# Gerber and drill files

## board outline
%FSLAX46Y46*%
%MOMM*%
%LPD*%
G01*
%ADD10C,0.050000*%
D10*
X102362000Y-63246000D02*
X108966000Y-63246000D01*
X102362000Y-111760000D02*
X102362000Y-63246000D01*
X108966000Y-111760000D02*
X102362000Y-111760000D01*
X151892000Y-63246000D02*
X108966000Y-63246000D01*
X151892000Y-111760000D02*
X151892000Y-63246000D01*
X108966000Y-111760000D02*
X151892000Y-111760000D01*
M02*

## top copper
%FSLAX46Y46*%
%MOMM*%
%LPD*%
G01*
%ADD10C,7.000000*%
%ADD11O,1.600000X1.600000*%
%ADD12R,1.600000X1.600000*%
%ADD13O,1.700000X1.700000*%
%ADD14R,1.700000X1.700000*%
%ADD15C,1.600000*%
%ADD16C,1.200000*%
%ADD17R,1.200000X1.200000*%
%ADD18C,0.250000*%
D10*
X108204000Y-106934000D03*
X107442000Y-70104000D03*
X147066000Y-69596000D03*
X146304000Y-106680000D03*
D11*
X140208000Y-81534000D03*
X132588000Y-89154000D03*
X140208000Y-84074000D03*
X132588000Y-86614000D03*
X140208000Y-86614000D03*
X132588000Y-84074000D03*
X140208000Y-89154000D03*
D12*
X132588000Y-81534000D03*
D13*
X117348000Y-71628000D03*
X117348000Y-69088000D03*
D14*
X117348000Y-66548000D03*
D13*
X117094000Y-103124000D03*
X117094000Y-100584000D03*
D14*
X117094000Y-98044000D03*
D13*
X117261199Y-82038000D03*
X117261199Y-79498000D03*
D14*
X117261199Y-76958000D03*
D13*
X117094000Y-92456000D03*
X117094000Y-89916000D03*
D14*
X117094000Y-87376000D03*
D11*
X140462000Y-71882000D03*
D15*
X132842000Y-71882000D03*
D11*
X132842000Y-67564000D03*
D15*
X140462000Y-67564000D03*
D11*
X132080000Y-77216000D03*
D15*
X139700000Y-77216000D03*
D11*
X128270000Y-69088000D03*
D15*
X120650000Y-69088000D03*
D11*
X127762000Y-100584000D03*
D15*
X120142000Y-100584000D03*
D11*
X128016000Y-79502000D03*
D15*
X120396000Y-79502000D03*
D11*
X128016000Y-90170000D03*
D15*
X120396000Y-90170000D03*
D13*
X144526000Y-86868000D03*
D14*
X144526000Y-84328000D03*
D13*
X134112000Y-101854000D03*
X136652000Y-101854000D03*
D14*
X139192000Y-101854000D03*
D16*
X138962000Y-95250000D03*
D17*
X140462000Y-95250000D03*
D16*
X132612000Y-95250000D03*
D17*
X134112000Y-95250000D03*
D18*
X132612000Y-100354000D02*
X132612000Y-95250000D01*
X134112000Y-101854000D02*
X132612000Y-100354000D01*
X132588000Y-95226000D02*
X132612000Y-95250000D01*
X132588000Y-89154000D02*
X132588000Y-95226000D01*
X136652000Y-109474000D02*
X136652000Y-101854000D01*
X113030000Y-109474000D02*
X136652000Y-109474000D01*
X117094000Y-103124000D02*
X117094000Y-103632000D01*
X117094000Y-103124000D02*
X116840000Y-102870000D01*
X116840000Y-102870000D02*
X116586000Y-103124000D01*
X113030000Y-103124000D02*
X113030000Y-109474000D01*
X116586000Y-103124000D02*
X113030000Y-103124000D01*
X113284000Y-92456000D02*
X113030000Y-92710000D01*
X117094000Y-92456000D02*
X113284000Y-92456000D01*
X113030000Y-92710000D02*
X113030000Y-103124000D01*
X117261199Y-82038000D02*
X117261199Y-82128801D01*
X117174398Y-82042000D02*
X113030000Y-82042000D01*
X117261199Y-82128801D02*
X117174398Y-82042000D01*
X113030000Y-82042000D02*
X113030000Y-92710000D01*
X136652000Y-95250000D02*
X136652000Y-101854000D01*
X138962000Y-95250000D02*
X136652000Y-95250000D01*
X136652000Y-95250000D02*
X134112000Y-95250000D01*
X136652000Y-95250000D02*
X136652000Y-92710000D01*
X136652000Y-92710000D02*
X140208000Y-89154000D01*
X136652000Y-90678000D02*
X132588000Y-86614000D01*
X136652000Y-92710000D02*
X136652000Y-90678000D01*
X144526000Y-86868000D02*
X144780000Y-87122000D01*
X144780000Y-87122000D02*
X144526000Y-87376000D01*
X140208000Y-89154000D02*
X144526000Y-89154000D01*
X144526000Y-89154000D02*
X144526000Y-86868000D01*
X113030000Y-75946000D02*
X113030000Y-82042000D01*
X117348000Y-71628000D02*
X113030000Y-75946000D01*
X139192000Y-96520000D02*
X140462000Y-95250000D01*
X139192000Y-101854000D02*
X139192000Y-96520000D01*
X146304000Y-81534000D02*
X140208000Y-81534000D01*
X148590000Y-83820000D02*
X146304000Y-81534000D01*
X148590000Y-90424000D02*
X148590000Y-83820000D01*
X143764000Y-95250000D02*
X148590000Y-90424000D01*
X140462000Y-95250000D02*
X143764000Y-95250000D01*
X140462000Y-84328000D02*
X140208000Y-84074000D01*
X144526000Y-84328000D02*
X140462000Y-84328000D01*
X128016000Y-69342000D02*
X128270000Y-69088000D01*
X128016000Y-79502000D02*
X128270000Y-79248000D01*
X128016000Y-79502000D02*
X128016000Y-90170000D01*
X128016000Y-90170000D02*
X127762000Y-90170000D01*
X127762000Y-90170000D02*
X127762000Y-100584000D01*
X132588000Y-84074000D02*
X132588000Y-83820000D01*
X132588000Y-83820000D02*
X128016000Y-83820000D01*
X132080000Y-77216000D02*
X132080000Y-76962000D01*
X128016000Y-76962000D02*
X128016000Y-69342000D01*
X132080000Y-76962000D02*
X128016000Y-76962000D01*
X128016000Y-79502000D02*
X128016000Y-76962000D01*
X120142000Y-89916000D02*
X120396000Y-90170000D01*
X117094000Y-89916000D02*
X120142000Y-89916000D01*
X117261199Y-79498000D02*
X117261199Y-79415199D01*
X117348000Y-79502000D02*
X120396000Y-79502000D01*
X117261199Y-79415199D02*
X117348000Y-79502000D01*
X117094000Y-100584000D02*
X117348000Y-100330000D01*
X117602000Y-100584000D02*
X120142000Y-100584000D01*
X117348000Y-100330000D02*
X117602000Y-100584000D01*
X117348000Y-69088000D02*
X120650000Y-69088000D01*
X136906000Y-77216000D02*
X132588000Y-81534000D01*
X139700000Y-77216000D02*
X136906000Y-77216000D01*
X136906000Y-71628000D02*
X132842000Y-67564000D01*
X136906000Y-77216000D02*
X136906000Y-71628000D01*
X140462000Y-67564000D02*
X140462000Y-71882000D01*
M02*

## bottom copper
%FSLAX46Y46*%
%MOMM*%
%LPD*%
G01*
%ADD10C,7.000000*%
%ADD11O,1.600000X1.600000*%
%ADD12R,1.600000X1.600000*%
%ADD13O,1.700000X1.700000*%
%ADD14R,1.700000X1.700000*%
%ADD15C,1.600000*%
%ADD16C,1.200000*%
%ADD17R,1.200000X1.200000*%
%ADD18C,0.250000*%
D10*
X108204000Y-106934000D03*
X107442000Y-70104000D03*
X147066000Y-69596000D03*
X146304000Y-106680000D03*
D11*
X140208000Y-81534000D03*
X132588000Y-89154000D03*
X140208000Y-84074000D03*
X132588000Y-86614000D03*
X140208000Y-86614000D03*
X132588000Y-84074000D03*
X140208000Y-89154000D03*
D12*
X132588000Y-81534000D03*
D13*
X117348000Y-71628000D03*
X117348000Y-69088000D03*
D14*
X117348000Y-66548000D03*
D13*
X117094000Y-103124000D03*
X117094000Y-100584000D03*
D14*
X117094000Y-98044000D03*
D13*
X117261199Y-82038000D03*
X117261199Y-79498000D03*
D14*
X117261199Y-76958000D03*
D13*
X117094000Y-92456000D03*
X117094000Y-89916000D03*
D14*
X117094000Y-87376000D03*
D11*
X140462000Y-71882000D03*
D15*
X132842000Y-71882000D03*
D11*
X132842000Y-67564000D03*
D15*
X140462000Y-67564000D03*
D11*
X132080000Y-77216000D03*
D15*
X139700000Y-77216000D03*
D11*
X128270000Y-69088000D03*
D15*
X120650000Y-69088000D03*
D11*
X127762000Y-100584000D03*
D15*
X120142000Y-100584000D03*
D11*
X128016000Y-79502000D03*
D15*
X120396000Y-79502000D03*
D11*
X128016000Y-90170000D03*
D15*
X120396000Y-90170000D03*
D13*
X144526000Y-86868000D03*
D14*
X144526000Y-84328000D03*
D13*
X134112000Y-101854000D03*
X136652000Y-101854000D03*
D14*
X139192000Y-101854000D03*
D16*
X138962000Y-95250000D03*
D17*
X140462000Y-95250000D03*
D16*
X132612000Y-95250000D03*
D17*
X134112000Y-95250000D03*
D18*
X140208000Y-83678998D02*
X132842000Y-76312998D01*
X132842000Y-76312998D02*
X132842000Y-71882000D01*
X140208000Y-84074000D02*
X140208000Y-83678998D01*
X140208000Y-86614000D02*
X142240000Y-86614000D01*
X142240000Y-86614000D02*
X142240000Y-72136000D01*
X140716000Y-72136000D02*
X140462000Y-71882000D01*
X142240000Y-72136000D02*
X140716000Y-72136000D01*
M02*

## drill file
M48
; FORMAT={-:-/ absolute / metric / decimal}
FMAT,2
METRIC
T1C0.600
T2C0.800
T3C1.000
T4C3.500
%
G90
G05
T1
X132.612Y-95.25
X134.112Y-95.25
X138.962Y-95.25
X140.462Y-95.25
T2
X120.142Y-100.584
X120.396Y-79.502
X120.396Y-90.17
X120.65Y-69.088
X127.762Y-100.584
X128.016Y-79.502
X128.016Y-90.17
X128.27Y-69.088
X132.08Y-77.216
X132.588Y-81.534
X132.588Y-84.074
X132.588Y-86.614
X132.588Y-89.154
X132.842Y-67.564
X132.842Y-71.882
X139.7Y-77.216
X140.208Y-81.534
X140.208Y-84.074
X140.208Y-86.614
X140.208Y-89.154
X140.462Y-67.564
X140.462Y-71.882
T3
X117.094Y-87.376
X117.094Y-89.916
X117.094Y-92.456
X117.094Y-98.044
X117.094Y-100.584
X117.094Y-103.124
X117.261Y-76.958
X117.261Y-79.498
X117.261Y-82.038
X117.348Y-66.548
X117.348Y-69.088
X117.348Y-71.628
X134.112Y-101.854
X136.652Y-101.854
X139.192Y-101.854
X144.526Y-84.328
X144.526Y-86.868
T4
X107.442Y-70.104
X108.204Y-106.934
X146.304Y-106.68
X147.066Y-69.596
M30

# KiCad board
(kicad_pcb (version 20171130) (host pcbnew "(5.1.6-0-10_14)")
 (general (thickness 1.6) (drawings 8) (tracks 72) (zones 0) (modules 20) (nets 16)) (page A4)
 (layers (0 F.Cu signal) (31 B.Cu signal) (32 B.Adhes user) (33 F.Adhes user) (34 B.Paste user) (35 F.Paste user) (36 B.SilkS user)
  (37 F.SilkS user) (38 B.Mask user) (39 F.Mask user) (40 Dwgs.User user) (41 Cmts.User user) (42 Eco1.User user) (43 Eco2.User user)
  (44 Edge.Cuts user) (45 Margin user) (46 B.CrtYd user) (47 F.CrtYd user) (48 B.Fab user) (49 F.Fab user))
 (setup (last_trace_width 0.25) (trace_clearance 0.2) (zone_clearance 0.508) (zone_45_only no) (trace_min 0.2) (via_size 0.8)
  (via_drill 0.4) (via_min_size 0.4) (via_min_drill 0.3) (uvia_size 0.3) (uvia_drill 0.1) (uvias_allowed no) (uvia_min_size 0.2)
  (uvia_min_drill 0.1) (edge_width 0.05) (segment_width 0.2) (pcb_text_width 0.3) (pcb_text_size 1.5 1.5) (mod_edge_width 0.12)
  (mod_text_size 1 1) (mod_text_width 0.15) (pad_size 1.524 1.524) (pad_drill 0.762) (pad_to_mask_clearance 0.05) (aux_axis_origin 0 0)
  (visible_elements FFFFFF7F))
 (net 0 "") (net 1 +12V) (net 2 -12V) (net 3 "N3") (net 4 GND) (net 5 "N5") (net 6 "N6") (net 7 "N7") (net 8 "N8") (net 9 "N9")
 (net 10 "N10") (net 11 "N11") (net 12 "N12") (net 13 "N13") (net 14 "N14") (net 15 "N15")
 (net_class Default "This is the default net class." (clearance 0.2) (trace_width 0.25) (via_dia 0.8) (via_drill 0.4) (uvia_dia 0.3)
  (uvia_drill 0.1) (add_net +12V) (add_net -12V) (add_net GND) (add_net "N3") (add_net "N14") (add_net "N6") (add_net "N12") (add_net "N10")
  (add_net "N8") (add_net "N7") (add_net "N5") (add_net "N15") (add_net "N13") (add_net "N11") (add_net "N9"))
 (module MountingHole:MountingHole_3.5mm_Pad (layer F.Cu) (at 108.204 106.934)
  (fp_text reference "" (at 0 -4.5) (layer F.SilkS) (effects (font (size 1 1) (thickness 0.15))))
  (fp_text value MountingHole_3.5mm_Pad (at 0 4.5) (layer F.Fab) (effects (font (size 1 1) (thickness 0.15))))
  (pad 1 thru_hole circle (at 0 0) (size 7 7) (drill 3.5) (layers *.Cu *.Mask)))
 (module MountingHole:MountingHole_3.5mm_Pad (layer F.Cu) (at 107.442 70.104)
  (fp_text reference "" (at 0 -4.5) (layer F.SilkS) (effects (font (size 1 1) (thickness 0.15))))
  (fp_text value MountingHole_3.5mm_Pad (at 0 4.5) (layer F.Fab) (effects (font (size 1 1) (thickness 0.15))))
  (pad 1 thru_hole circle (at 0 0) (size 7 7) (drill 3.5) (layers *.Cu *.Mask)))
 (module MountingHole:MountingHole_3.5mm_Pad (layer F.Cu) (at 147.066 69.596)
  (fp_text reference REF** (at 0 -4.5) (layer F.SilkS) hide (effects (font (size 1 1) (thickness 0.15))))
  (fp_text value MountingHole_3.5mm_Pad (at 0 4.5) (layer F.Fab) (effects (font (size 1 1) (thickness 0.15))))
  (pad 1 thru_hole circle (at 0 0) (size 7 7) (drill 3.5) (layers *.Cu *.Mask)))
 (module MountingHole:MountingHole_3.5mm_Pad (layer F.Cu) (at 146.304 106.68)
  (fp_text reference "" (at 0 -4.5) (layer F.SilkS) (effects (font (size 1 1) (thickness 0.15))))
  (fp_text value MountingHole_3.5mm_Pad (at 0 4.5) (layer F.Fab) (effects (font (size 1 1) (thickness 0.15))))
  (pad 1 thru_hole circle (at 0 0) (size 7 7) (drill 3.5) (layers *.Cu *.Mask)))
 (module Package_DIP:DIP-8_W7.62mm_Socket (layer F.Cu) (at 132.588 81.534)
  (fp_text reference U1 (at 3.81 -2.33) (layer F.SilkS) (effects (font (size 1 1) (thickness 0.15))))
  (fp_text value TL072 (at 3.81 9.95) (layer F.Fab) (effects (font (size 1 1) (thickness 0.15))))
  (pad 8 thru_hole oval (at 7.62 0) (size 1.6 1.6) (drill 0.8) (layers *.Cu *.Mask) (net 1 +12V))
  (pad 4 thru_hole oval (at 0 7.62) (size 1.6 1.6) (drill 0.8) (layers *.Cu *.Mask) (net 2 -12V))
  (pad 7 thru_hole oval (at 7.62 2.54) (size 1.6 1.6) (drill 0.8) (layers *.Cu *.Mask) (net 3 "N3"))
  (pad 3 thru_hole oval (at 0 5.08) (size 1.6 1.6) (drill 0.8) (layers *.Cu *.Mask) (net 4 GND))
  (pad 6 thru_hole oval (at 7.62 5.08) (size 1.6 1.6) (drill 0.8) (layers *.Cu *.Mask) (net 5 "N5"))
  (pad 2 thru_hole oval (at 0 2.54) (size 1.6 1.6) (drill 0.8) (layers *.Cu *.Mask) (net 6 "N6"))
  (pad 5 thru_hole oval (at 7.62 7.62) (size 1.6 1.6) (drill 0.8) (layers *.Cu *.Mask) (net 4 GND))
  (pad 1 thru_hole rect (at 0 0) (size 1.6 1.6) (drill 0.8) (layers *.Cu *.Mask) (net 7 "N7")))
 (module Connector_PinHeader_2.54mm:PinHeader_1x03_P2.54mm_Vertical (layer F.Cu) (at 117.348 66.548)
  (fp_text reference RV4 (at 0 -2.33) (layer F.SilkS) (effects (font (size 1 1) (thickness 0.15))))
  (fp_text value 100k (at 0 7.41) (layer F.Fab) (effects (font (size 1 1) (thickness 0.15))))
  (pad 3 thru_hole oval (at 0 5.08) (size 1.7 1.7) (drill 1) (layers *.Cu *.Mask) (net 4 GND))
  (pad 2 thru_hole oval (at 0 2.54) (size 1.7 1.7) (drill 1) (layers *.Cu *.Mask) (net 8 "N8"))
  (pad 1 thru_hole rect (at 0 0) (size 1.7 1.7) (drill 1) (layers *.Cu *.Mask) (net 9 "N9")))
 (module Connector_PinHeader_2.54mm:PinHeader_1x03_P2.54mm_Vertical (layer F.Cu) (at 117.094 98.044)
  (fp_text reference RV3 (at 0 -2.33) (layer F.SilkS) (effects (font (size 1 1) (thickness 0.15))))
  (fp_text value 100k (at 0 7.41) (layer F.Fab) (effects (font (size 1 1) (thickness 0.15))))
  (pad 3 thru_hole oval (at 0 5.08) (size 1.7 1.7) (drill 1) (layers *.Cu *.Mask) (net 4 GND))
  (pad 2 thru_hole oval (at 0 2.54) (size 1.7 1.7) (drill 1) (layers *.Cu *.Mask) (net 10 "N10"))
  (pad 1 thru_hole rect (at 0 0) (size 1.7 1.7) (drill 1) (layers *.Cu *.Mask) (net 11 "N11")))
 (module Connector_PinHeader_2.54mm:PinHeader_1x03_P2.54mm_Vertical (layer F.Cu) (at 117.261199 76.958)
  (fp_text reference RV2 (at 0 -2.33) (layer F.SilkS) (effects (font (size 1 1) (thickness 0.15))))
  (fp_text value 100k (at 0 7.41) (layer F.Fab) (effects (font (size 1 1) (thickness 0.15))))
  (pad 3 thru_hole oval (at 0 5.08) (size 1.7 1.7) (drill 1) (layers *.Cu *.Mask) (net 4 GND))
  (pad 2 thru_hole oval (at 0 2.54) (size 1.7 1.7) (drill 1) (layers *.Cu *.Mask) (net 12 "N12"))
  (pad 1 thru_hole rect (at 0 0) (size 1.7 1.7) (drill 1) (layers *.Cu *.Mask) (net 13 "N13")))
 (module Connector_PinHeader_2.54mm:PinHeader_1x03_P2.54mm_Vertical (layer F.Cu) (at 117.094 87.376)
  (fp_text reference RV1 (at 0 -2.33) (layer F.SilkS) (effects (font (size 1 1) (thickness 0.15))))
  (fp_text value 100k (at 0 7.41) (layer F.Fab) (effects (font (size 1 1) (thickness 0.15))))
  (pad 3 thru_hole oval (at 0 5.08) (size 1.7 1.7) (drill 1) (layers *.Cu *.Mask) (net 4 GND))
  (pad 2 thru_hole oval (at 0 2.54) (size 1.7 1.7) (drill 1) (layers *.Cu *.Mask) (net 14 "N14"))
  (pad 1 thru_hole rect (at 0 0) (size 1.7 1.7) (drill 1) (layers *.Cu *.Mask) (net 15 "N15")))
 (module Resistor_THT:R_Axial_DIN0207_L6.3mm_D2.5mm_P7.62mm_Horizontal (layer F.Cu) (at 132.842 71.882)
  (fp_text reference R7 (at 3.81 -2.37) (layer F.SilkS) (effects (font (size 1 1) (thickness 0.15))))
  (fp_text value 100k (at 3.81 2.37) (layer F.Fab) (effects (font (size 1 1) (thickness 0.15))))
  (pad 2 thru_hole oval (at 7.62 0) (size 1.6 1.6) (drill 0.8) (layers *.Cu *.Mask) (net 5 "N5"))
  (pad 1 thru_hole circle (at 0 0) (size 1.6 1.6) (drill 0.8) (layers *.Cu *.Mask) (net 3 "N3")))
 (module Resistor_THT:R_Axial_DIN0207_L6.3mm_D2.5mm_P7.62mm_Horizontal (layer F.Cu) (at 140.462 67.564 180)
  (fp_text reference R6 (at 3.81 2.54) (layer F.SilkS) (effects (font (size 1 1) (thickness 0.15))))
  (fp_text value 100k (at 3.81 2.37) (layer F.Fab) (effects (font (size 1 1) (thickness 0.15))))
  (pad 2 thru_hole oval (at 7.62 0 180) (size 1.6 1.6) (drill 0.8) (layers *.Cu *.Mask) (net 7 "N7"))
  (pad 1 thru_hole circle (at 0 0 180) (size 1.6 1.6) (drill 0.8) (layers *.Cu *.Mask) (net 5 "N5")))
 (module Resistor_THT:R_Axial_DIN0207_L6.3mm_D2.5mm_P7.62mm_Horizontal (layer F.Cu) (at 139.7 77.216 180)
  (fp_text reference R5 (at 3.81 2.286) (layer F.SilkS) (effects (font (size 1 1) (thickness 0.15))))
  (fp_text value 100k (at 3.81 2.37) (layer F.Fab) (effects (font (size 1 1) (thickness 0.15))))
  (pad 2 thru_hole oval (at 7.62 0 180) (size 1.6 1.6) (drill 0.8) (layers *.Cu *.Mask) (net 6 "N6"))
  (pad 1 thru_hole circle (at 0 0 180) (size 1.6 1.6) (drill 0.8) (layers *.Cu *.Mask) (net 7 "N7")))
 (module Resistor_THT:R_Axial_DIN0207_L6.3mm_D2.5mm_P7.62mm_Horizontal (layer F.Cu) (at 120.65 69.088)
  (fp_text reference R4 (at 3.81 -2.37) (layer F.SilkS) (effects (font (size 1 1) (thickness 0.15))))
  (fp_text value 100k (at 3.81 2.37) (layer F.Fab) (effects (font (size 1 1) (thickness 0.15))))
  (pad 2 thru_hole oval (at 7.62 0) (size 1.6 1.6) (drill 0.8) (layers *.Cu *.Mask) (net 6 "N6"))
  (pad 1 thru_hole circle (at 0 0) (size 1.6 1.6) (drill 0.8) (layers *.Cu *.Mask) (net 8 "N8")))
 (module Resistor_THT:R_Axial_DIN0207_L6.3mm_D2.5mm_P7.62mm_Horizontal (layer F.Cu) (at 120.142 100.584)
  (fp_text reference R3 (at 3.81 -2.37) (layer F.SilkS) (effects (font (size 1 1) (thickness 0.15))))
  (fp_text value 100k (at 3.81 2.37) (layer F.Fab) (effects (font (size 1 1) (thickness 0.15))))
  (pad 2 thru_hole oval (at 7.62 0) (size 1.6 1.6) (drill 0.8) (layers *.Cu *.Mask) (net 6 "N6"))
  (pad 1 thru_hole circle (at 0 0) (size 1.6 1.6) (drill 0.8) (layers *.Cu *.Mask) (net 10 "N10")))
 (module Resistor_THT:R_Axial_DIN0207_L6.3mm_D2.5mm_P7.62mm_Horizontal (layer F.Cu) (at 120.396 79.502)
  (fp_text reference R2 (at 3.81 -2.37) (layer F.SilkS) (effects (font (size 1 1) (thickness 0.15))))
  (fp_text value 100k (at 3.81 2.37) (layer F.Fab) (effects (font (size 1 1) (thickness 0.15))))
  (pad 2 thru_hole oval (at 7.62 0) (size 1.6 1.6) (drill 0.8) (layers *.Cu *.Mask) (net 6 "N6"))
  (pad 1 thru_hole circle (at 0 0) (size 1.6 1.6) (drill 0.8) (layers *.Cu *.Mask) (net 12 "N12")))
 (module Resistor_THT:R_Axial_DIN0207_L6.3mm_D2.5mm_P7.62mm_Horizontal (layer F.Cu) (at 120.396 90.17)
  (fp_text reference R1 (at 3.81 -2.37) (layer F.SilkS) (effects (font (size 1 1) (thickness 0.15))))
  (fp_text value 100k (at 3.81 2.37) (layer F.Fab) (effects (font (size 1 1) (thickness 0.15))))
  (pad 2 thru_hole oval (at 7.62 0) (size 1.6 1.6) (drill 0.8) (layers *.Cu *.Mask) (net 6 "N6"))
  (pad 1 thru_hole circle (at 0 0) (size 1.6 1.6) (drill 0.8) (layers *.Cu *.Mask) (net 14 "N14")))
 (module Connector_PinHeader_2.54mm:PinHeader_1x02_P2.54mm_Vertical (layer F.Cu) (at 144.526 84.328)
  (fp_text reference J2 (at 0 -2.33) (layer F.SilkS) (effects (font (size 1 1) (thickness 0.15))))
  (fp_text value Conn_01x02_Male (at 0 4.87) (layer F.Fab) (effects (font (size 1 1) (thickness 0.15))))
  (pad 2 thru_hole oval (at 0 2.54) (size 1.7 1.7) (drill 1) (layers *.Cu *.Mask) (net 4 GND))
  (pad 1 thru_hole rect (at 0 0) (size 1.7 1.7) (drill 1) (layers *.Cu *.Mask) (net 3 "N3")))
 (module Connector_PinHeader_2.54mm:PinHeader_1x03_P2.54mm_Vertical (layer F.Cu) (at 139.192 101.854 270)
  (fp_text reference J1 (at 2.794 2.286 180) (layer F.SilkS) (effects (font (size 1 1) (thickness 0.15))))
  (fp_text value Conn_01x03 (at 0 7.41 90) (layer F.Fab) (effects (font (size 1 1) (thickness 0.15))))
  (pad 3 thru_hole oval (at 0 5.08 270) (size 1.7 1.7) (drill 1) (layers *.Cu *.Mask) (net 2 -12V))
  (pad 2 thru_hole oval (at 0 2.54 270) (size 1.7 1.7) (drill 1) (layers *.Cu *.Mask) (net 4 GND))
  (pad 1 thru_hole rect (at 0 0 270) (size 1.7 1.7) (drill 1) (layers *.Cu *.Mask) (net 1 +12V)))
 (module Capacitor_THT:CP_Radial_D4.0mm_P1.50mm (layer F.Cu) (at 140.462 95.25 180)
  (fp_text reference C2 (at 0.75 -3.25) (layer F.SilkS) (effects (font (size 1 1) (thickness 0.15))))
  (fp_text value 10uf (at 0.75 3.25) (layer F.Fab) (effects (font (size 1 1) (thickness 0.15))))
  (pad 2 thru_hole circle (at 1.5 0 180) (size 1.2 1.2) (drill 0.6) (layers *.Cu *.Mask) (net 4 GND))
  (pad 1 thru_hole rect (at 0 0 180) (size 1.2 1.2) (drill 0.6) (layers *.Cu *.Mask) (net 1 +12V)))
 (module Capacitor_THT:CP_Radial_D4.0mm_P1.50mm (layer F.Cu) (at 134.112 95.25 180)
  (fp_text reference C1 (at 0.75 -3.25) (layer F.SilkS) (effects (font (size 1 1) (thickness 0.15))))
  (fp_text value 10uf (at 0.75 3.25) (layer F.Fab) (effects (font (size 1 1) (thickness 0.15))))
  (pad 2 thru_hole circle (at 1.5 0 180) (size 1.2 1.2) (drill 0.6) (layers *.Cu *.Mask) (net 2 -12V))
  (pad 1 thru_hole rect (at 0 0 180) (size 1.2 1.2) (drill 0.6) (layers *.Cu *.Mask) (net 4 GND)))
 (gr_line (start 102.362 63.246) (end 108.966 63.246) (layer Edge.Cuts) (width 0.05))
 (gr_line (start 102.362 111.76) (end 102.362 63.246) (layer Edge.Cuts) (width 0.05))
 (gr_line (start 108.966 111.76) (end 102.362 111.76) (layer Edge.Cuts) (width 0.05))
 (gr_line (start 151.892 63.246) (end 108.966 63.246) (layer Edge.Cuts) (width 0.05))
 (gr_line (start 151.892 111.76) (end 151.892 63.246) (layer Edge.Cuts) (width 0.05))
 (gr_line (start 108.966 111.76) (end 151.892 111.76) (layer Edge.Cuts) (width 0.05))
 (segment (start 132.612 100.354) (end 132.612 95.25) (width 0.25) (layer F.Cu) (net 2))
 (segment (start 134.112 101.854) (end 132.612 100.354) (width 0.25) (layer F.Cu) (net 2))
 (segment (start 132.588 95.226) (end 132.612 95.25) (width 0.25) (layer F.Cu) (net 2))
 (segment (start 132.588 89.154) (end 132.588 95.226) (width 0.25) (layer F.Cu) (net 2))
 (segment (start 136.652 109.474) (end 136.652 101.854) (width 0.25) (layer F.Cu) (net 4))
 (segment (start 113.03 109.474) (end 136.652 109.474) (width 0.25) (layer F.Cu) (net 4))
 (segment (start 117.094 103.124) (end 117.094 103.632) (width 0.25) (layer F.Cu) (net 4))
 (segment (start 117.094 103.124) (end 116.84 102.87) (width 0.25) (layer F.Cu) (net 4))
 (segment (start 116.84 102.87) (end 116.586 103.124) (width 0.25) (layer F.Cu) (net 4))
 (segment (start 113.03 103.124) (end 113.03 109.474) (width 0.25) (layer F.Cu) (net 4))
 (segment (start 116.586 103.124) (end 113.03 103.124) (width 0.25) (layer F.Cu) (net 4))
 (segment (start 113.284 92.456) (end 113.03 92.71) (width 0.25) (layer F.Cu) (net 4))
 (segment (start 117.094 92.456) (end 113.284 92.456) (width 0.25) (layer F.Cu) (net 4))
 (segment (start 113.03 92.71) (end 113.03 103.124) (width 0.25) (layer F.Cu) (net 4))
 (segment (start 117.261199 82.038) (end 117.261199 82.128801) (width 0.25) (layer F.Cu) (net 4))
 (segment (start 117.174398 82.042) (end 113.03 82.042) (width 0.25) (layer F.Cu) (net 4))
 (segment (start 117.261199 82.128801) (end 117.174398 82.042) (width 0.25) (layer F.Cu) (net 4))
 (segment (start 113.03 82.042) (end 113.03 92.71) (width 0.25) (layer F.Cu) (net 4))
 (segment (start 136.652 95.25) (end 136.652 101.854) (width 0.25) (layer F.Cu) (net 4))
 (segment (start 138.962 95.25) (end 136.652 95.25) (width 0.25) (layer F.Cu) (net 4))
 (segment (start 136.652 95.25) (end 134.112 95.25) (width 0.25) (layer F.Cu) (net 4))
 (segment (start 136.652 95.25) (end 136.652 92.71) (width 0.25) (layer F.Cu) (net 4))
 (segment (start 136.652 92.71) (end 140.208 89.154) (width 0.25) (layer F.Cu) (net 4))
 (segment (start 136.652 90.678) (end 132.588 86.614) (width 0.25) (layer F.Cu) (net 4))
 (segment (start 136.652 92.71) (end 136.652 90.678) (width 0.25) (layer F.Cu) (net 4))
 (segment (start 144.526 86.868) (end 144.78 87.122) (width 0.25) (layer F.Cu) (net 4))
 (segment (start 144.78 87.122) (end 144.526 87.376) (width 0.25) (layer F.Cu) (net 4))
 (segment (start 140.208 89.154) (end 144.526 89.154) (width 0.25) (layer F.Cu) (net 4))
 (segment (start 144.526 89.154) (end 144.526 86.868) (width 0.25) (layer F.Cu) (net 4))
 (segment (start 113.03 75.946) (end 113.03 82.042) (width 0.25) (layer F.Cu) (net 4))
 (segment (start 117.348 71.628) (end 113.03 75.946) (width 0.25) (layer F.Cu) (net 4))
 (segment (start 139.192 96.52) (end 140.462 95.25) (width 0.25) (layer F.Cu) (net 1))
 (segment (start 139.192 101.854) (end 139.192 96.52) (width 0.25) (layer F.Cu) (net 1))
 (segment (start 146.304 81.534) (end 140.208 81.534) (width 0.25) (layer F.Cu) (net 1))
 (segment (start 148.59 83.82) (end 146.304 81.534) (width 0.25) (layer F.Cu) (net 1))
 (segment (start 148.59 90.424) (end 148.59 83.82) (width 0.25) (layer F.Cu) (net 1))
 (segment (start 143.764 95.25) (end 148.59 90.424) (width 0.25) (layer F.Cu) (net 1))
 (segment (start 140.462 95.25) (end 143.764 95.25) (width 0.25) (layer F.Cu) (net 1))
 (segment (start 140.462 84.328) (end 140.208 84.074) (width 0.25) (layer F.Cu) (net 3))
 (segment (start 144.526 84.328) (end 140.462 84.328) (width 0.25) (layer F.Cu) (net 3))
 (segment (start 140.208 83.678998) (end 132.842 76.312998) (width 0.25) (layer B.Cu) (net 3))
 (segment (start 132.842 76.312998) (end 132.842 71.882) (width 0.25) (layer B.Cu) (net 3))
 (segment (start 140.208 84.074) (end 140.208 83.678998) (width 0.25) (layer B.Cu) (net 3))
 (segment (start 128.016 69.342) (end 128.27 69.088) (width 0.25) (layer F.Cu) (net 6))
 (segment (start 128.016 79.502) (end 128.27 79.248) (width 0.25) (layer F.Cu) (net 6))
 (segment (start 128.016 79.502) (end 128.016 90.17) (width 0.25) (layer F.Cu) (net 6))
 (segment (start 128.016 90.17) (end 127.762 90.17) (width 0.25) (layer F.Cu) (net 6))
 (segment (start 127.762 90.17) (end 127.762 100.584) (width 0.25) (layer F.Cu) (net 6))
 (segment (start 132.588 84.074) (end 132.588 83.82) (width 0.25) (layer F.Cu) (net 6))
 (segment (start 132.588 83.82) (end 128.016 83.82) (width 0.25) (layer F.Cu) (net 6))
 (segment (start 132.08 77.216) (end 132.08 76.962) (width 0.25) (layer F.Cu) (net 6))
 (segment (start 128.016 76.962) (end 128.016 69.342) (width 0.25) (layer F.Cu) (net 6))
 (segment (start 132.08 76.962) (end 128.016 76.962) (width 0.25) (layer F.Cu) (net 6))
 (segment (start 128.016 79.502) (end 128.016 76.962) (width 0.25) (layer F.Cu) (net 6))
 (segment (start 120.142 89.916) (end 120.396 90.17) (width 0.25) (layer F.Cu) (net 14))
 (segment (start 117.094 89.916) (end 120.142 89.916) (width 0.25) (layer F.Cu) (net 14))
 (segment (start 117.261199 79.498) (end 117.261199 79.415199) (width 0.25) (layer F.Cu) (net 12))
 (segment (start 117.348 79.502) (end 120.396 79.502) (width 0.25) (layer F.Cu) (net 12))
 (segment (start 117.261199 79.415199) (end 117.348 79.502) (width 0.25) (layer F.Cu) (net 12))
 (segment (start 117.094 100.584) (end 117.348 100.33) (width 0.25) (layer F.Cu) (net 10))
 (segment (start 117.602 100.584) (end 120.142 100.584) (width 0.25) (layer F.Cu) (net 10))
 (segment (start 117.348 100.33) (end 117.602 100.584) (width 0.25) (layer F.Cu) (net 10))
 (segment (start 117.348 69.088) (end 120.65 69.088) (width 0.25) (layer F.Cu) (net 8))
 (segment (start 136.906 77.216) (end 132.588 81.534) (width 0.25) (layer F.Cu) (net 7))
 (segment (start 139.7 77.216) (end 136.906 77.216) (width 0.25) (layer F.Cu) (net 7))
 (segment (start 136.906 71.628) (end 132.842 67.564) (width 0.25) (layer F.Cu) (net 7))
 (segment (start 136.906 77.216) (end 136.906 71.628) (width 0.25) (layer F.Cu) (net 7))
 (segment (start 140.462 67.564) (end 140.462 71.882) (width 0.25) (layer F.Cu) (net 5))
 (segment (start 140.208 86.614) (end 142.24 86.614) (width 0.25) (layer B.Cu) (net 5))
 (segment (start 142.24 86.614) (end 142.24 72.136) (width 0.25) (layer B.Cu) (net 5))
 (segment (start 140.716 72.136) (end 140.462 71.882) (width 0.25) (layer B.Cu) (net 5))
 (segment (start 142.24 72.136) (end 140.716 72.136) (width 0.25) (layer B.Cu) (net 5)))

